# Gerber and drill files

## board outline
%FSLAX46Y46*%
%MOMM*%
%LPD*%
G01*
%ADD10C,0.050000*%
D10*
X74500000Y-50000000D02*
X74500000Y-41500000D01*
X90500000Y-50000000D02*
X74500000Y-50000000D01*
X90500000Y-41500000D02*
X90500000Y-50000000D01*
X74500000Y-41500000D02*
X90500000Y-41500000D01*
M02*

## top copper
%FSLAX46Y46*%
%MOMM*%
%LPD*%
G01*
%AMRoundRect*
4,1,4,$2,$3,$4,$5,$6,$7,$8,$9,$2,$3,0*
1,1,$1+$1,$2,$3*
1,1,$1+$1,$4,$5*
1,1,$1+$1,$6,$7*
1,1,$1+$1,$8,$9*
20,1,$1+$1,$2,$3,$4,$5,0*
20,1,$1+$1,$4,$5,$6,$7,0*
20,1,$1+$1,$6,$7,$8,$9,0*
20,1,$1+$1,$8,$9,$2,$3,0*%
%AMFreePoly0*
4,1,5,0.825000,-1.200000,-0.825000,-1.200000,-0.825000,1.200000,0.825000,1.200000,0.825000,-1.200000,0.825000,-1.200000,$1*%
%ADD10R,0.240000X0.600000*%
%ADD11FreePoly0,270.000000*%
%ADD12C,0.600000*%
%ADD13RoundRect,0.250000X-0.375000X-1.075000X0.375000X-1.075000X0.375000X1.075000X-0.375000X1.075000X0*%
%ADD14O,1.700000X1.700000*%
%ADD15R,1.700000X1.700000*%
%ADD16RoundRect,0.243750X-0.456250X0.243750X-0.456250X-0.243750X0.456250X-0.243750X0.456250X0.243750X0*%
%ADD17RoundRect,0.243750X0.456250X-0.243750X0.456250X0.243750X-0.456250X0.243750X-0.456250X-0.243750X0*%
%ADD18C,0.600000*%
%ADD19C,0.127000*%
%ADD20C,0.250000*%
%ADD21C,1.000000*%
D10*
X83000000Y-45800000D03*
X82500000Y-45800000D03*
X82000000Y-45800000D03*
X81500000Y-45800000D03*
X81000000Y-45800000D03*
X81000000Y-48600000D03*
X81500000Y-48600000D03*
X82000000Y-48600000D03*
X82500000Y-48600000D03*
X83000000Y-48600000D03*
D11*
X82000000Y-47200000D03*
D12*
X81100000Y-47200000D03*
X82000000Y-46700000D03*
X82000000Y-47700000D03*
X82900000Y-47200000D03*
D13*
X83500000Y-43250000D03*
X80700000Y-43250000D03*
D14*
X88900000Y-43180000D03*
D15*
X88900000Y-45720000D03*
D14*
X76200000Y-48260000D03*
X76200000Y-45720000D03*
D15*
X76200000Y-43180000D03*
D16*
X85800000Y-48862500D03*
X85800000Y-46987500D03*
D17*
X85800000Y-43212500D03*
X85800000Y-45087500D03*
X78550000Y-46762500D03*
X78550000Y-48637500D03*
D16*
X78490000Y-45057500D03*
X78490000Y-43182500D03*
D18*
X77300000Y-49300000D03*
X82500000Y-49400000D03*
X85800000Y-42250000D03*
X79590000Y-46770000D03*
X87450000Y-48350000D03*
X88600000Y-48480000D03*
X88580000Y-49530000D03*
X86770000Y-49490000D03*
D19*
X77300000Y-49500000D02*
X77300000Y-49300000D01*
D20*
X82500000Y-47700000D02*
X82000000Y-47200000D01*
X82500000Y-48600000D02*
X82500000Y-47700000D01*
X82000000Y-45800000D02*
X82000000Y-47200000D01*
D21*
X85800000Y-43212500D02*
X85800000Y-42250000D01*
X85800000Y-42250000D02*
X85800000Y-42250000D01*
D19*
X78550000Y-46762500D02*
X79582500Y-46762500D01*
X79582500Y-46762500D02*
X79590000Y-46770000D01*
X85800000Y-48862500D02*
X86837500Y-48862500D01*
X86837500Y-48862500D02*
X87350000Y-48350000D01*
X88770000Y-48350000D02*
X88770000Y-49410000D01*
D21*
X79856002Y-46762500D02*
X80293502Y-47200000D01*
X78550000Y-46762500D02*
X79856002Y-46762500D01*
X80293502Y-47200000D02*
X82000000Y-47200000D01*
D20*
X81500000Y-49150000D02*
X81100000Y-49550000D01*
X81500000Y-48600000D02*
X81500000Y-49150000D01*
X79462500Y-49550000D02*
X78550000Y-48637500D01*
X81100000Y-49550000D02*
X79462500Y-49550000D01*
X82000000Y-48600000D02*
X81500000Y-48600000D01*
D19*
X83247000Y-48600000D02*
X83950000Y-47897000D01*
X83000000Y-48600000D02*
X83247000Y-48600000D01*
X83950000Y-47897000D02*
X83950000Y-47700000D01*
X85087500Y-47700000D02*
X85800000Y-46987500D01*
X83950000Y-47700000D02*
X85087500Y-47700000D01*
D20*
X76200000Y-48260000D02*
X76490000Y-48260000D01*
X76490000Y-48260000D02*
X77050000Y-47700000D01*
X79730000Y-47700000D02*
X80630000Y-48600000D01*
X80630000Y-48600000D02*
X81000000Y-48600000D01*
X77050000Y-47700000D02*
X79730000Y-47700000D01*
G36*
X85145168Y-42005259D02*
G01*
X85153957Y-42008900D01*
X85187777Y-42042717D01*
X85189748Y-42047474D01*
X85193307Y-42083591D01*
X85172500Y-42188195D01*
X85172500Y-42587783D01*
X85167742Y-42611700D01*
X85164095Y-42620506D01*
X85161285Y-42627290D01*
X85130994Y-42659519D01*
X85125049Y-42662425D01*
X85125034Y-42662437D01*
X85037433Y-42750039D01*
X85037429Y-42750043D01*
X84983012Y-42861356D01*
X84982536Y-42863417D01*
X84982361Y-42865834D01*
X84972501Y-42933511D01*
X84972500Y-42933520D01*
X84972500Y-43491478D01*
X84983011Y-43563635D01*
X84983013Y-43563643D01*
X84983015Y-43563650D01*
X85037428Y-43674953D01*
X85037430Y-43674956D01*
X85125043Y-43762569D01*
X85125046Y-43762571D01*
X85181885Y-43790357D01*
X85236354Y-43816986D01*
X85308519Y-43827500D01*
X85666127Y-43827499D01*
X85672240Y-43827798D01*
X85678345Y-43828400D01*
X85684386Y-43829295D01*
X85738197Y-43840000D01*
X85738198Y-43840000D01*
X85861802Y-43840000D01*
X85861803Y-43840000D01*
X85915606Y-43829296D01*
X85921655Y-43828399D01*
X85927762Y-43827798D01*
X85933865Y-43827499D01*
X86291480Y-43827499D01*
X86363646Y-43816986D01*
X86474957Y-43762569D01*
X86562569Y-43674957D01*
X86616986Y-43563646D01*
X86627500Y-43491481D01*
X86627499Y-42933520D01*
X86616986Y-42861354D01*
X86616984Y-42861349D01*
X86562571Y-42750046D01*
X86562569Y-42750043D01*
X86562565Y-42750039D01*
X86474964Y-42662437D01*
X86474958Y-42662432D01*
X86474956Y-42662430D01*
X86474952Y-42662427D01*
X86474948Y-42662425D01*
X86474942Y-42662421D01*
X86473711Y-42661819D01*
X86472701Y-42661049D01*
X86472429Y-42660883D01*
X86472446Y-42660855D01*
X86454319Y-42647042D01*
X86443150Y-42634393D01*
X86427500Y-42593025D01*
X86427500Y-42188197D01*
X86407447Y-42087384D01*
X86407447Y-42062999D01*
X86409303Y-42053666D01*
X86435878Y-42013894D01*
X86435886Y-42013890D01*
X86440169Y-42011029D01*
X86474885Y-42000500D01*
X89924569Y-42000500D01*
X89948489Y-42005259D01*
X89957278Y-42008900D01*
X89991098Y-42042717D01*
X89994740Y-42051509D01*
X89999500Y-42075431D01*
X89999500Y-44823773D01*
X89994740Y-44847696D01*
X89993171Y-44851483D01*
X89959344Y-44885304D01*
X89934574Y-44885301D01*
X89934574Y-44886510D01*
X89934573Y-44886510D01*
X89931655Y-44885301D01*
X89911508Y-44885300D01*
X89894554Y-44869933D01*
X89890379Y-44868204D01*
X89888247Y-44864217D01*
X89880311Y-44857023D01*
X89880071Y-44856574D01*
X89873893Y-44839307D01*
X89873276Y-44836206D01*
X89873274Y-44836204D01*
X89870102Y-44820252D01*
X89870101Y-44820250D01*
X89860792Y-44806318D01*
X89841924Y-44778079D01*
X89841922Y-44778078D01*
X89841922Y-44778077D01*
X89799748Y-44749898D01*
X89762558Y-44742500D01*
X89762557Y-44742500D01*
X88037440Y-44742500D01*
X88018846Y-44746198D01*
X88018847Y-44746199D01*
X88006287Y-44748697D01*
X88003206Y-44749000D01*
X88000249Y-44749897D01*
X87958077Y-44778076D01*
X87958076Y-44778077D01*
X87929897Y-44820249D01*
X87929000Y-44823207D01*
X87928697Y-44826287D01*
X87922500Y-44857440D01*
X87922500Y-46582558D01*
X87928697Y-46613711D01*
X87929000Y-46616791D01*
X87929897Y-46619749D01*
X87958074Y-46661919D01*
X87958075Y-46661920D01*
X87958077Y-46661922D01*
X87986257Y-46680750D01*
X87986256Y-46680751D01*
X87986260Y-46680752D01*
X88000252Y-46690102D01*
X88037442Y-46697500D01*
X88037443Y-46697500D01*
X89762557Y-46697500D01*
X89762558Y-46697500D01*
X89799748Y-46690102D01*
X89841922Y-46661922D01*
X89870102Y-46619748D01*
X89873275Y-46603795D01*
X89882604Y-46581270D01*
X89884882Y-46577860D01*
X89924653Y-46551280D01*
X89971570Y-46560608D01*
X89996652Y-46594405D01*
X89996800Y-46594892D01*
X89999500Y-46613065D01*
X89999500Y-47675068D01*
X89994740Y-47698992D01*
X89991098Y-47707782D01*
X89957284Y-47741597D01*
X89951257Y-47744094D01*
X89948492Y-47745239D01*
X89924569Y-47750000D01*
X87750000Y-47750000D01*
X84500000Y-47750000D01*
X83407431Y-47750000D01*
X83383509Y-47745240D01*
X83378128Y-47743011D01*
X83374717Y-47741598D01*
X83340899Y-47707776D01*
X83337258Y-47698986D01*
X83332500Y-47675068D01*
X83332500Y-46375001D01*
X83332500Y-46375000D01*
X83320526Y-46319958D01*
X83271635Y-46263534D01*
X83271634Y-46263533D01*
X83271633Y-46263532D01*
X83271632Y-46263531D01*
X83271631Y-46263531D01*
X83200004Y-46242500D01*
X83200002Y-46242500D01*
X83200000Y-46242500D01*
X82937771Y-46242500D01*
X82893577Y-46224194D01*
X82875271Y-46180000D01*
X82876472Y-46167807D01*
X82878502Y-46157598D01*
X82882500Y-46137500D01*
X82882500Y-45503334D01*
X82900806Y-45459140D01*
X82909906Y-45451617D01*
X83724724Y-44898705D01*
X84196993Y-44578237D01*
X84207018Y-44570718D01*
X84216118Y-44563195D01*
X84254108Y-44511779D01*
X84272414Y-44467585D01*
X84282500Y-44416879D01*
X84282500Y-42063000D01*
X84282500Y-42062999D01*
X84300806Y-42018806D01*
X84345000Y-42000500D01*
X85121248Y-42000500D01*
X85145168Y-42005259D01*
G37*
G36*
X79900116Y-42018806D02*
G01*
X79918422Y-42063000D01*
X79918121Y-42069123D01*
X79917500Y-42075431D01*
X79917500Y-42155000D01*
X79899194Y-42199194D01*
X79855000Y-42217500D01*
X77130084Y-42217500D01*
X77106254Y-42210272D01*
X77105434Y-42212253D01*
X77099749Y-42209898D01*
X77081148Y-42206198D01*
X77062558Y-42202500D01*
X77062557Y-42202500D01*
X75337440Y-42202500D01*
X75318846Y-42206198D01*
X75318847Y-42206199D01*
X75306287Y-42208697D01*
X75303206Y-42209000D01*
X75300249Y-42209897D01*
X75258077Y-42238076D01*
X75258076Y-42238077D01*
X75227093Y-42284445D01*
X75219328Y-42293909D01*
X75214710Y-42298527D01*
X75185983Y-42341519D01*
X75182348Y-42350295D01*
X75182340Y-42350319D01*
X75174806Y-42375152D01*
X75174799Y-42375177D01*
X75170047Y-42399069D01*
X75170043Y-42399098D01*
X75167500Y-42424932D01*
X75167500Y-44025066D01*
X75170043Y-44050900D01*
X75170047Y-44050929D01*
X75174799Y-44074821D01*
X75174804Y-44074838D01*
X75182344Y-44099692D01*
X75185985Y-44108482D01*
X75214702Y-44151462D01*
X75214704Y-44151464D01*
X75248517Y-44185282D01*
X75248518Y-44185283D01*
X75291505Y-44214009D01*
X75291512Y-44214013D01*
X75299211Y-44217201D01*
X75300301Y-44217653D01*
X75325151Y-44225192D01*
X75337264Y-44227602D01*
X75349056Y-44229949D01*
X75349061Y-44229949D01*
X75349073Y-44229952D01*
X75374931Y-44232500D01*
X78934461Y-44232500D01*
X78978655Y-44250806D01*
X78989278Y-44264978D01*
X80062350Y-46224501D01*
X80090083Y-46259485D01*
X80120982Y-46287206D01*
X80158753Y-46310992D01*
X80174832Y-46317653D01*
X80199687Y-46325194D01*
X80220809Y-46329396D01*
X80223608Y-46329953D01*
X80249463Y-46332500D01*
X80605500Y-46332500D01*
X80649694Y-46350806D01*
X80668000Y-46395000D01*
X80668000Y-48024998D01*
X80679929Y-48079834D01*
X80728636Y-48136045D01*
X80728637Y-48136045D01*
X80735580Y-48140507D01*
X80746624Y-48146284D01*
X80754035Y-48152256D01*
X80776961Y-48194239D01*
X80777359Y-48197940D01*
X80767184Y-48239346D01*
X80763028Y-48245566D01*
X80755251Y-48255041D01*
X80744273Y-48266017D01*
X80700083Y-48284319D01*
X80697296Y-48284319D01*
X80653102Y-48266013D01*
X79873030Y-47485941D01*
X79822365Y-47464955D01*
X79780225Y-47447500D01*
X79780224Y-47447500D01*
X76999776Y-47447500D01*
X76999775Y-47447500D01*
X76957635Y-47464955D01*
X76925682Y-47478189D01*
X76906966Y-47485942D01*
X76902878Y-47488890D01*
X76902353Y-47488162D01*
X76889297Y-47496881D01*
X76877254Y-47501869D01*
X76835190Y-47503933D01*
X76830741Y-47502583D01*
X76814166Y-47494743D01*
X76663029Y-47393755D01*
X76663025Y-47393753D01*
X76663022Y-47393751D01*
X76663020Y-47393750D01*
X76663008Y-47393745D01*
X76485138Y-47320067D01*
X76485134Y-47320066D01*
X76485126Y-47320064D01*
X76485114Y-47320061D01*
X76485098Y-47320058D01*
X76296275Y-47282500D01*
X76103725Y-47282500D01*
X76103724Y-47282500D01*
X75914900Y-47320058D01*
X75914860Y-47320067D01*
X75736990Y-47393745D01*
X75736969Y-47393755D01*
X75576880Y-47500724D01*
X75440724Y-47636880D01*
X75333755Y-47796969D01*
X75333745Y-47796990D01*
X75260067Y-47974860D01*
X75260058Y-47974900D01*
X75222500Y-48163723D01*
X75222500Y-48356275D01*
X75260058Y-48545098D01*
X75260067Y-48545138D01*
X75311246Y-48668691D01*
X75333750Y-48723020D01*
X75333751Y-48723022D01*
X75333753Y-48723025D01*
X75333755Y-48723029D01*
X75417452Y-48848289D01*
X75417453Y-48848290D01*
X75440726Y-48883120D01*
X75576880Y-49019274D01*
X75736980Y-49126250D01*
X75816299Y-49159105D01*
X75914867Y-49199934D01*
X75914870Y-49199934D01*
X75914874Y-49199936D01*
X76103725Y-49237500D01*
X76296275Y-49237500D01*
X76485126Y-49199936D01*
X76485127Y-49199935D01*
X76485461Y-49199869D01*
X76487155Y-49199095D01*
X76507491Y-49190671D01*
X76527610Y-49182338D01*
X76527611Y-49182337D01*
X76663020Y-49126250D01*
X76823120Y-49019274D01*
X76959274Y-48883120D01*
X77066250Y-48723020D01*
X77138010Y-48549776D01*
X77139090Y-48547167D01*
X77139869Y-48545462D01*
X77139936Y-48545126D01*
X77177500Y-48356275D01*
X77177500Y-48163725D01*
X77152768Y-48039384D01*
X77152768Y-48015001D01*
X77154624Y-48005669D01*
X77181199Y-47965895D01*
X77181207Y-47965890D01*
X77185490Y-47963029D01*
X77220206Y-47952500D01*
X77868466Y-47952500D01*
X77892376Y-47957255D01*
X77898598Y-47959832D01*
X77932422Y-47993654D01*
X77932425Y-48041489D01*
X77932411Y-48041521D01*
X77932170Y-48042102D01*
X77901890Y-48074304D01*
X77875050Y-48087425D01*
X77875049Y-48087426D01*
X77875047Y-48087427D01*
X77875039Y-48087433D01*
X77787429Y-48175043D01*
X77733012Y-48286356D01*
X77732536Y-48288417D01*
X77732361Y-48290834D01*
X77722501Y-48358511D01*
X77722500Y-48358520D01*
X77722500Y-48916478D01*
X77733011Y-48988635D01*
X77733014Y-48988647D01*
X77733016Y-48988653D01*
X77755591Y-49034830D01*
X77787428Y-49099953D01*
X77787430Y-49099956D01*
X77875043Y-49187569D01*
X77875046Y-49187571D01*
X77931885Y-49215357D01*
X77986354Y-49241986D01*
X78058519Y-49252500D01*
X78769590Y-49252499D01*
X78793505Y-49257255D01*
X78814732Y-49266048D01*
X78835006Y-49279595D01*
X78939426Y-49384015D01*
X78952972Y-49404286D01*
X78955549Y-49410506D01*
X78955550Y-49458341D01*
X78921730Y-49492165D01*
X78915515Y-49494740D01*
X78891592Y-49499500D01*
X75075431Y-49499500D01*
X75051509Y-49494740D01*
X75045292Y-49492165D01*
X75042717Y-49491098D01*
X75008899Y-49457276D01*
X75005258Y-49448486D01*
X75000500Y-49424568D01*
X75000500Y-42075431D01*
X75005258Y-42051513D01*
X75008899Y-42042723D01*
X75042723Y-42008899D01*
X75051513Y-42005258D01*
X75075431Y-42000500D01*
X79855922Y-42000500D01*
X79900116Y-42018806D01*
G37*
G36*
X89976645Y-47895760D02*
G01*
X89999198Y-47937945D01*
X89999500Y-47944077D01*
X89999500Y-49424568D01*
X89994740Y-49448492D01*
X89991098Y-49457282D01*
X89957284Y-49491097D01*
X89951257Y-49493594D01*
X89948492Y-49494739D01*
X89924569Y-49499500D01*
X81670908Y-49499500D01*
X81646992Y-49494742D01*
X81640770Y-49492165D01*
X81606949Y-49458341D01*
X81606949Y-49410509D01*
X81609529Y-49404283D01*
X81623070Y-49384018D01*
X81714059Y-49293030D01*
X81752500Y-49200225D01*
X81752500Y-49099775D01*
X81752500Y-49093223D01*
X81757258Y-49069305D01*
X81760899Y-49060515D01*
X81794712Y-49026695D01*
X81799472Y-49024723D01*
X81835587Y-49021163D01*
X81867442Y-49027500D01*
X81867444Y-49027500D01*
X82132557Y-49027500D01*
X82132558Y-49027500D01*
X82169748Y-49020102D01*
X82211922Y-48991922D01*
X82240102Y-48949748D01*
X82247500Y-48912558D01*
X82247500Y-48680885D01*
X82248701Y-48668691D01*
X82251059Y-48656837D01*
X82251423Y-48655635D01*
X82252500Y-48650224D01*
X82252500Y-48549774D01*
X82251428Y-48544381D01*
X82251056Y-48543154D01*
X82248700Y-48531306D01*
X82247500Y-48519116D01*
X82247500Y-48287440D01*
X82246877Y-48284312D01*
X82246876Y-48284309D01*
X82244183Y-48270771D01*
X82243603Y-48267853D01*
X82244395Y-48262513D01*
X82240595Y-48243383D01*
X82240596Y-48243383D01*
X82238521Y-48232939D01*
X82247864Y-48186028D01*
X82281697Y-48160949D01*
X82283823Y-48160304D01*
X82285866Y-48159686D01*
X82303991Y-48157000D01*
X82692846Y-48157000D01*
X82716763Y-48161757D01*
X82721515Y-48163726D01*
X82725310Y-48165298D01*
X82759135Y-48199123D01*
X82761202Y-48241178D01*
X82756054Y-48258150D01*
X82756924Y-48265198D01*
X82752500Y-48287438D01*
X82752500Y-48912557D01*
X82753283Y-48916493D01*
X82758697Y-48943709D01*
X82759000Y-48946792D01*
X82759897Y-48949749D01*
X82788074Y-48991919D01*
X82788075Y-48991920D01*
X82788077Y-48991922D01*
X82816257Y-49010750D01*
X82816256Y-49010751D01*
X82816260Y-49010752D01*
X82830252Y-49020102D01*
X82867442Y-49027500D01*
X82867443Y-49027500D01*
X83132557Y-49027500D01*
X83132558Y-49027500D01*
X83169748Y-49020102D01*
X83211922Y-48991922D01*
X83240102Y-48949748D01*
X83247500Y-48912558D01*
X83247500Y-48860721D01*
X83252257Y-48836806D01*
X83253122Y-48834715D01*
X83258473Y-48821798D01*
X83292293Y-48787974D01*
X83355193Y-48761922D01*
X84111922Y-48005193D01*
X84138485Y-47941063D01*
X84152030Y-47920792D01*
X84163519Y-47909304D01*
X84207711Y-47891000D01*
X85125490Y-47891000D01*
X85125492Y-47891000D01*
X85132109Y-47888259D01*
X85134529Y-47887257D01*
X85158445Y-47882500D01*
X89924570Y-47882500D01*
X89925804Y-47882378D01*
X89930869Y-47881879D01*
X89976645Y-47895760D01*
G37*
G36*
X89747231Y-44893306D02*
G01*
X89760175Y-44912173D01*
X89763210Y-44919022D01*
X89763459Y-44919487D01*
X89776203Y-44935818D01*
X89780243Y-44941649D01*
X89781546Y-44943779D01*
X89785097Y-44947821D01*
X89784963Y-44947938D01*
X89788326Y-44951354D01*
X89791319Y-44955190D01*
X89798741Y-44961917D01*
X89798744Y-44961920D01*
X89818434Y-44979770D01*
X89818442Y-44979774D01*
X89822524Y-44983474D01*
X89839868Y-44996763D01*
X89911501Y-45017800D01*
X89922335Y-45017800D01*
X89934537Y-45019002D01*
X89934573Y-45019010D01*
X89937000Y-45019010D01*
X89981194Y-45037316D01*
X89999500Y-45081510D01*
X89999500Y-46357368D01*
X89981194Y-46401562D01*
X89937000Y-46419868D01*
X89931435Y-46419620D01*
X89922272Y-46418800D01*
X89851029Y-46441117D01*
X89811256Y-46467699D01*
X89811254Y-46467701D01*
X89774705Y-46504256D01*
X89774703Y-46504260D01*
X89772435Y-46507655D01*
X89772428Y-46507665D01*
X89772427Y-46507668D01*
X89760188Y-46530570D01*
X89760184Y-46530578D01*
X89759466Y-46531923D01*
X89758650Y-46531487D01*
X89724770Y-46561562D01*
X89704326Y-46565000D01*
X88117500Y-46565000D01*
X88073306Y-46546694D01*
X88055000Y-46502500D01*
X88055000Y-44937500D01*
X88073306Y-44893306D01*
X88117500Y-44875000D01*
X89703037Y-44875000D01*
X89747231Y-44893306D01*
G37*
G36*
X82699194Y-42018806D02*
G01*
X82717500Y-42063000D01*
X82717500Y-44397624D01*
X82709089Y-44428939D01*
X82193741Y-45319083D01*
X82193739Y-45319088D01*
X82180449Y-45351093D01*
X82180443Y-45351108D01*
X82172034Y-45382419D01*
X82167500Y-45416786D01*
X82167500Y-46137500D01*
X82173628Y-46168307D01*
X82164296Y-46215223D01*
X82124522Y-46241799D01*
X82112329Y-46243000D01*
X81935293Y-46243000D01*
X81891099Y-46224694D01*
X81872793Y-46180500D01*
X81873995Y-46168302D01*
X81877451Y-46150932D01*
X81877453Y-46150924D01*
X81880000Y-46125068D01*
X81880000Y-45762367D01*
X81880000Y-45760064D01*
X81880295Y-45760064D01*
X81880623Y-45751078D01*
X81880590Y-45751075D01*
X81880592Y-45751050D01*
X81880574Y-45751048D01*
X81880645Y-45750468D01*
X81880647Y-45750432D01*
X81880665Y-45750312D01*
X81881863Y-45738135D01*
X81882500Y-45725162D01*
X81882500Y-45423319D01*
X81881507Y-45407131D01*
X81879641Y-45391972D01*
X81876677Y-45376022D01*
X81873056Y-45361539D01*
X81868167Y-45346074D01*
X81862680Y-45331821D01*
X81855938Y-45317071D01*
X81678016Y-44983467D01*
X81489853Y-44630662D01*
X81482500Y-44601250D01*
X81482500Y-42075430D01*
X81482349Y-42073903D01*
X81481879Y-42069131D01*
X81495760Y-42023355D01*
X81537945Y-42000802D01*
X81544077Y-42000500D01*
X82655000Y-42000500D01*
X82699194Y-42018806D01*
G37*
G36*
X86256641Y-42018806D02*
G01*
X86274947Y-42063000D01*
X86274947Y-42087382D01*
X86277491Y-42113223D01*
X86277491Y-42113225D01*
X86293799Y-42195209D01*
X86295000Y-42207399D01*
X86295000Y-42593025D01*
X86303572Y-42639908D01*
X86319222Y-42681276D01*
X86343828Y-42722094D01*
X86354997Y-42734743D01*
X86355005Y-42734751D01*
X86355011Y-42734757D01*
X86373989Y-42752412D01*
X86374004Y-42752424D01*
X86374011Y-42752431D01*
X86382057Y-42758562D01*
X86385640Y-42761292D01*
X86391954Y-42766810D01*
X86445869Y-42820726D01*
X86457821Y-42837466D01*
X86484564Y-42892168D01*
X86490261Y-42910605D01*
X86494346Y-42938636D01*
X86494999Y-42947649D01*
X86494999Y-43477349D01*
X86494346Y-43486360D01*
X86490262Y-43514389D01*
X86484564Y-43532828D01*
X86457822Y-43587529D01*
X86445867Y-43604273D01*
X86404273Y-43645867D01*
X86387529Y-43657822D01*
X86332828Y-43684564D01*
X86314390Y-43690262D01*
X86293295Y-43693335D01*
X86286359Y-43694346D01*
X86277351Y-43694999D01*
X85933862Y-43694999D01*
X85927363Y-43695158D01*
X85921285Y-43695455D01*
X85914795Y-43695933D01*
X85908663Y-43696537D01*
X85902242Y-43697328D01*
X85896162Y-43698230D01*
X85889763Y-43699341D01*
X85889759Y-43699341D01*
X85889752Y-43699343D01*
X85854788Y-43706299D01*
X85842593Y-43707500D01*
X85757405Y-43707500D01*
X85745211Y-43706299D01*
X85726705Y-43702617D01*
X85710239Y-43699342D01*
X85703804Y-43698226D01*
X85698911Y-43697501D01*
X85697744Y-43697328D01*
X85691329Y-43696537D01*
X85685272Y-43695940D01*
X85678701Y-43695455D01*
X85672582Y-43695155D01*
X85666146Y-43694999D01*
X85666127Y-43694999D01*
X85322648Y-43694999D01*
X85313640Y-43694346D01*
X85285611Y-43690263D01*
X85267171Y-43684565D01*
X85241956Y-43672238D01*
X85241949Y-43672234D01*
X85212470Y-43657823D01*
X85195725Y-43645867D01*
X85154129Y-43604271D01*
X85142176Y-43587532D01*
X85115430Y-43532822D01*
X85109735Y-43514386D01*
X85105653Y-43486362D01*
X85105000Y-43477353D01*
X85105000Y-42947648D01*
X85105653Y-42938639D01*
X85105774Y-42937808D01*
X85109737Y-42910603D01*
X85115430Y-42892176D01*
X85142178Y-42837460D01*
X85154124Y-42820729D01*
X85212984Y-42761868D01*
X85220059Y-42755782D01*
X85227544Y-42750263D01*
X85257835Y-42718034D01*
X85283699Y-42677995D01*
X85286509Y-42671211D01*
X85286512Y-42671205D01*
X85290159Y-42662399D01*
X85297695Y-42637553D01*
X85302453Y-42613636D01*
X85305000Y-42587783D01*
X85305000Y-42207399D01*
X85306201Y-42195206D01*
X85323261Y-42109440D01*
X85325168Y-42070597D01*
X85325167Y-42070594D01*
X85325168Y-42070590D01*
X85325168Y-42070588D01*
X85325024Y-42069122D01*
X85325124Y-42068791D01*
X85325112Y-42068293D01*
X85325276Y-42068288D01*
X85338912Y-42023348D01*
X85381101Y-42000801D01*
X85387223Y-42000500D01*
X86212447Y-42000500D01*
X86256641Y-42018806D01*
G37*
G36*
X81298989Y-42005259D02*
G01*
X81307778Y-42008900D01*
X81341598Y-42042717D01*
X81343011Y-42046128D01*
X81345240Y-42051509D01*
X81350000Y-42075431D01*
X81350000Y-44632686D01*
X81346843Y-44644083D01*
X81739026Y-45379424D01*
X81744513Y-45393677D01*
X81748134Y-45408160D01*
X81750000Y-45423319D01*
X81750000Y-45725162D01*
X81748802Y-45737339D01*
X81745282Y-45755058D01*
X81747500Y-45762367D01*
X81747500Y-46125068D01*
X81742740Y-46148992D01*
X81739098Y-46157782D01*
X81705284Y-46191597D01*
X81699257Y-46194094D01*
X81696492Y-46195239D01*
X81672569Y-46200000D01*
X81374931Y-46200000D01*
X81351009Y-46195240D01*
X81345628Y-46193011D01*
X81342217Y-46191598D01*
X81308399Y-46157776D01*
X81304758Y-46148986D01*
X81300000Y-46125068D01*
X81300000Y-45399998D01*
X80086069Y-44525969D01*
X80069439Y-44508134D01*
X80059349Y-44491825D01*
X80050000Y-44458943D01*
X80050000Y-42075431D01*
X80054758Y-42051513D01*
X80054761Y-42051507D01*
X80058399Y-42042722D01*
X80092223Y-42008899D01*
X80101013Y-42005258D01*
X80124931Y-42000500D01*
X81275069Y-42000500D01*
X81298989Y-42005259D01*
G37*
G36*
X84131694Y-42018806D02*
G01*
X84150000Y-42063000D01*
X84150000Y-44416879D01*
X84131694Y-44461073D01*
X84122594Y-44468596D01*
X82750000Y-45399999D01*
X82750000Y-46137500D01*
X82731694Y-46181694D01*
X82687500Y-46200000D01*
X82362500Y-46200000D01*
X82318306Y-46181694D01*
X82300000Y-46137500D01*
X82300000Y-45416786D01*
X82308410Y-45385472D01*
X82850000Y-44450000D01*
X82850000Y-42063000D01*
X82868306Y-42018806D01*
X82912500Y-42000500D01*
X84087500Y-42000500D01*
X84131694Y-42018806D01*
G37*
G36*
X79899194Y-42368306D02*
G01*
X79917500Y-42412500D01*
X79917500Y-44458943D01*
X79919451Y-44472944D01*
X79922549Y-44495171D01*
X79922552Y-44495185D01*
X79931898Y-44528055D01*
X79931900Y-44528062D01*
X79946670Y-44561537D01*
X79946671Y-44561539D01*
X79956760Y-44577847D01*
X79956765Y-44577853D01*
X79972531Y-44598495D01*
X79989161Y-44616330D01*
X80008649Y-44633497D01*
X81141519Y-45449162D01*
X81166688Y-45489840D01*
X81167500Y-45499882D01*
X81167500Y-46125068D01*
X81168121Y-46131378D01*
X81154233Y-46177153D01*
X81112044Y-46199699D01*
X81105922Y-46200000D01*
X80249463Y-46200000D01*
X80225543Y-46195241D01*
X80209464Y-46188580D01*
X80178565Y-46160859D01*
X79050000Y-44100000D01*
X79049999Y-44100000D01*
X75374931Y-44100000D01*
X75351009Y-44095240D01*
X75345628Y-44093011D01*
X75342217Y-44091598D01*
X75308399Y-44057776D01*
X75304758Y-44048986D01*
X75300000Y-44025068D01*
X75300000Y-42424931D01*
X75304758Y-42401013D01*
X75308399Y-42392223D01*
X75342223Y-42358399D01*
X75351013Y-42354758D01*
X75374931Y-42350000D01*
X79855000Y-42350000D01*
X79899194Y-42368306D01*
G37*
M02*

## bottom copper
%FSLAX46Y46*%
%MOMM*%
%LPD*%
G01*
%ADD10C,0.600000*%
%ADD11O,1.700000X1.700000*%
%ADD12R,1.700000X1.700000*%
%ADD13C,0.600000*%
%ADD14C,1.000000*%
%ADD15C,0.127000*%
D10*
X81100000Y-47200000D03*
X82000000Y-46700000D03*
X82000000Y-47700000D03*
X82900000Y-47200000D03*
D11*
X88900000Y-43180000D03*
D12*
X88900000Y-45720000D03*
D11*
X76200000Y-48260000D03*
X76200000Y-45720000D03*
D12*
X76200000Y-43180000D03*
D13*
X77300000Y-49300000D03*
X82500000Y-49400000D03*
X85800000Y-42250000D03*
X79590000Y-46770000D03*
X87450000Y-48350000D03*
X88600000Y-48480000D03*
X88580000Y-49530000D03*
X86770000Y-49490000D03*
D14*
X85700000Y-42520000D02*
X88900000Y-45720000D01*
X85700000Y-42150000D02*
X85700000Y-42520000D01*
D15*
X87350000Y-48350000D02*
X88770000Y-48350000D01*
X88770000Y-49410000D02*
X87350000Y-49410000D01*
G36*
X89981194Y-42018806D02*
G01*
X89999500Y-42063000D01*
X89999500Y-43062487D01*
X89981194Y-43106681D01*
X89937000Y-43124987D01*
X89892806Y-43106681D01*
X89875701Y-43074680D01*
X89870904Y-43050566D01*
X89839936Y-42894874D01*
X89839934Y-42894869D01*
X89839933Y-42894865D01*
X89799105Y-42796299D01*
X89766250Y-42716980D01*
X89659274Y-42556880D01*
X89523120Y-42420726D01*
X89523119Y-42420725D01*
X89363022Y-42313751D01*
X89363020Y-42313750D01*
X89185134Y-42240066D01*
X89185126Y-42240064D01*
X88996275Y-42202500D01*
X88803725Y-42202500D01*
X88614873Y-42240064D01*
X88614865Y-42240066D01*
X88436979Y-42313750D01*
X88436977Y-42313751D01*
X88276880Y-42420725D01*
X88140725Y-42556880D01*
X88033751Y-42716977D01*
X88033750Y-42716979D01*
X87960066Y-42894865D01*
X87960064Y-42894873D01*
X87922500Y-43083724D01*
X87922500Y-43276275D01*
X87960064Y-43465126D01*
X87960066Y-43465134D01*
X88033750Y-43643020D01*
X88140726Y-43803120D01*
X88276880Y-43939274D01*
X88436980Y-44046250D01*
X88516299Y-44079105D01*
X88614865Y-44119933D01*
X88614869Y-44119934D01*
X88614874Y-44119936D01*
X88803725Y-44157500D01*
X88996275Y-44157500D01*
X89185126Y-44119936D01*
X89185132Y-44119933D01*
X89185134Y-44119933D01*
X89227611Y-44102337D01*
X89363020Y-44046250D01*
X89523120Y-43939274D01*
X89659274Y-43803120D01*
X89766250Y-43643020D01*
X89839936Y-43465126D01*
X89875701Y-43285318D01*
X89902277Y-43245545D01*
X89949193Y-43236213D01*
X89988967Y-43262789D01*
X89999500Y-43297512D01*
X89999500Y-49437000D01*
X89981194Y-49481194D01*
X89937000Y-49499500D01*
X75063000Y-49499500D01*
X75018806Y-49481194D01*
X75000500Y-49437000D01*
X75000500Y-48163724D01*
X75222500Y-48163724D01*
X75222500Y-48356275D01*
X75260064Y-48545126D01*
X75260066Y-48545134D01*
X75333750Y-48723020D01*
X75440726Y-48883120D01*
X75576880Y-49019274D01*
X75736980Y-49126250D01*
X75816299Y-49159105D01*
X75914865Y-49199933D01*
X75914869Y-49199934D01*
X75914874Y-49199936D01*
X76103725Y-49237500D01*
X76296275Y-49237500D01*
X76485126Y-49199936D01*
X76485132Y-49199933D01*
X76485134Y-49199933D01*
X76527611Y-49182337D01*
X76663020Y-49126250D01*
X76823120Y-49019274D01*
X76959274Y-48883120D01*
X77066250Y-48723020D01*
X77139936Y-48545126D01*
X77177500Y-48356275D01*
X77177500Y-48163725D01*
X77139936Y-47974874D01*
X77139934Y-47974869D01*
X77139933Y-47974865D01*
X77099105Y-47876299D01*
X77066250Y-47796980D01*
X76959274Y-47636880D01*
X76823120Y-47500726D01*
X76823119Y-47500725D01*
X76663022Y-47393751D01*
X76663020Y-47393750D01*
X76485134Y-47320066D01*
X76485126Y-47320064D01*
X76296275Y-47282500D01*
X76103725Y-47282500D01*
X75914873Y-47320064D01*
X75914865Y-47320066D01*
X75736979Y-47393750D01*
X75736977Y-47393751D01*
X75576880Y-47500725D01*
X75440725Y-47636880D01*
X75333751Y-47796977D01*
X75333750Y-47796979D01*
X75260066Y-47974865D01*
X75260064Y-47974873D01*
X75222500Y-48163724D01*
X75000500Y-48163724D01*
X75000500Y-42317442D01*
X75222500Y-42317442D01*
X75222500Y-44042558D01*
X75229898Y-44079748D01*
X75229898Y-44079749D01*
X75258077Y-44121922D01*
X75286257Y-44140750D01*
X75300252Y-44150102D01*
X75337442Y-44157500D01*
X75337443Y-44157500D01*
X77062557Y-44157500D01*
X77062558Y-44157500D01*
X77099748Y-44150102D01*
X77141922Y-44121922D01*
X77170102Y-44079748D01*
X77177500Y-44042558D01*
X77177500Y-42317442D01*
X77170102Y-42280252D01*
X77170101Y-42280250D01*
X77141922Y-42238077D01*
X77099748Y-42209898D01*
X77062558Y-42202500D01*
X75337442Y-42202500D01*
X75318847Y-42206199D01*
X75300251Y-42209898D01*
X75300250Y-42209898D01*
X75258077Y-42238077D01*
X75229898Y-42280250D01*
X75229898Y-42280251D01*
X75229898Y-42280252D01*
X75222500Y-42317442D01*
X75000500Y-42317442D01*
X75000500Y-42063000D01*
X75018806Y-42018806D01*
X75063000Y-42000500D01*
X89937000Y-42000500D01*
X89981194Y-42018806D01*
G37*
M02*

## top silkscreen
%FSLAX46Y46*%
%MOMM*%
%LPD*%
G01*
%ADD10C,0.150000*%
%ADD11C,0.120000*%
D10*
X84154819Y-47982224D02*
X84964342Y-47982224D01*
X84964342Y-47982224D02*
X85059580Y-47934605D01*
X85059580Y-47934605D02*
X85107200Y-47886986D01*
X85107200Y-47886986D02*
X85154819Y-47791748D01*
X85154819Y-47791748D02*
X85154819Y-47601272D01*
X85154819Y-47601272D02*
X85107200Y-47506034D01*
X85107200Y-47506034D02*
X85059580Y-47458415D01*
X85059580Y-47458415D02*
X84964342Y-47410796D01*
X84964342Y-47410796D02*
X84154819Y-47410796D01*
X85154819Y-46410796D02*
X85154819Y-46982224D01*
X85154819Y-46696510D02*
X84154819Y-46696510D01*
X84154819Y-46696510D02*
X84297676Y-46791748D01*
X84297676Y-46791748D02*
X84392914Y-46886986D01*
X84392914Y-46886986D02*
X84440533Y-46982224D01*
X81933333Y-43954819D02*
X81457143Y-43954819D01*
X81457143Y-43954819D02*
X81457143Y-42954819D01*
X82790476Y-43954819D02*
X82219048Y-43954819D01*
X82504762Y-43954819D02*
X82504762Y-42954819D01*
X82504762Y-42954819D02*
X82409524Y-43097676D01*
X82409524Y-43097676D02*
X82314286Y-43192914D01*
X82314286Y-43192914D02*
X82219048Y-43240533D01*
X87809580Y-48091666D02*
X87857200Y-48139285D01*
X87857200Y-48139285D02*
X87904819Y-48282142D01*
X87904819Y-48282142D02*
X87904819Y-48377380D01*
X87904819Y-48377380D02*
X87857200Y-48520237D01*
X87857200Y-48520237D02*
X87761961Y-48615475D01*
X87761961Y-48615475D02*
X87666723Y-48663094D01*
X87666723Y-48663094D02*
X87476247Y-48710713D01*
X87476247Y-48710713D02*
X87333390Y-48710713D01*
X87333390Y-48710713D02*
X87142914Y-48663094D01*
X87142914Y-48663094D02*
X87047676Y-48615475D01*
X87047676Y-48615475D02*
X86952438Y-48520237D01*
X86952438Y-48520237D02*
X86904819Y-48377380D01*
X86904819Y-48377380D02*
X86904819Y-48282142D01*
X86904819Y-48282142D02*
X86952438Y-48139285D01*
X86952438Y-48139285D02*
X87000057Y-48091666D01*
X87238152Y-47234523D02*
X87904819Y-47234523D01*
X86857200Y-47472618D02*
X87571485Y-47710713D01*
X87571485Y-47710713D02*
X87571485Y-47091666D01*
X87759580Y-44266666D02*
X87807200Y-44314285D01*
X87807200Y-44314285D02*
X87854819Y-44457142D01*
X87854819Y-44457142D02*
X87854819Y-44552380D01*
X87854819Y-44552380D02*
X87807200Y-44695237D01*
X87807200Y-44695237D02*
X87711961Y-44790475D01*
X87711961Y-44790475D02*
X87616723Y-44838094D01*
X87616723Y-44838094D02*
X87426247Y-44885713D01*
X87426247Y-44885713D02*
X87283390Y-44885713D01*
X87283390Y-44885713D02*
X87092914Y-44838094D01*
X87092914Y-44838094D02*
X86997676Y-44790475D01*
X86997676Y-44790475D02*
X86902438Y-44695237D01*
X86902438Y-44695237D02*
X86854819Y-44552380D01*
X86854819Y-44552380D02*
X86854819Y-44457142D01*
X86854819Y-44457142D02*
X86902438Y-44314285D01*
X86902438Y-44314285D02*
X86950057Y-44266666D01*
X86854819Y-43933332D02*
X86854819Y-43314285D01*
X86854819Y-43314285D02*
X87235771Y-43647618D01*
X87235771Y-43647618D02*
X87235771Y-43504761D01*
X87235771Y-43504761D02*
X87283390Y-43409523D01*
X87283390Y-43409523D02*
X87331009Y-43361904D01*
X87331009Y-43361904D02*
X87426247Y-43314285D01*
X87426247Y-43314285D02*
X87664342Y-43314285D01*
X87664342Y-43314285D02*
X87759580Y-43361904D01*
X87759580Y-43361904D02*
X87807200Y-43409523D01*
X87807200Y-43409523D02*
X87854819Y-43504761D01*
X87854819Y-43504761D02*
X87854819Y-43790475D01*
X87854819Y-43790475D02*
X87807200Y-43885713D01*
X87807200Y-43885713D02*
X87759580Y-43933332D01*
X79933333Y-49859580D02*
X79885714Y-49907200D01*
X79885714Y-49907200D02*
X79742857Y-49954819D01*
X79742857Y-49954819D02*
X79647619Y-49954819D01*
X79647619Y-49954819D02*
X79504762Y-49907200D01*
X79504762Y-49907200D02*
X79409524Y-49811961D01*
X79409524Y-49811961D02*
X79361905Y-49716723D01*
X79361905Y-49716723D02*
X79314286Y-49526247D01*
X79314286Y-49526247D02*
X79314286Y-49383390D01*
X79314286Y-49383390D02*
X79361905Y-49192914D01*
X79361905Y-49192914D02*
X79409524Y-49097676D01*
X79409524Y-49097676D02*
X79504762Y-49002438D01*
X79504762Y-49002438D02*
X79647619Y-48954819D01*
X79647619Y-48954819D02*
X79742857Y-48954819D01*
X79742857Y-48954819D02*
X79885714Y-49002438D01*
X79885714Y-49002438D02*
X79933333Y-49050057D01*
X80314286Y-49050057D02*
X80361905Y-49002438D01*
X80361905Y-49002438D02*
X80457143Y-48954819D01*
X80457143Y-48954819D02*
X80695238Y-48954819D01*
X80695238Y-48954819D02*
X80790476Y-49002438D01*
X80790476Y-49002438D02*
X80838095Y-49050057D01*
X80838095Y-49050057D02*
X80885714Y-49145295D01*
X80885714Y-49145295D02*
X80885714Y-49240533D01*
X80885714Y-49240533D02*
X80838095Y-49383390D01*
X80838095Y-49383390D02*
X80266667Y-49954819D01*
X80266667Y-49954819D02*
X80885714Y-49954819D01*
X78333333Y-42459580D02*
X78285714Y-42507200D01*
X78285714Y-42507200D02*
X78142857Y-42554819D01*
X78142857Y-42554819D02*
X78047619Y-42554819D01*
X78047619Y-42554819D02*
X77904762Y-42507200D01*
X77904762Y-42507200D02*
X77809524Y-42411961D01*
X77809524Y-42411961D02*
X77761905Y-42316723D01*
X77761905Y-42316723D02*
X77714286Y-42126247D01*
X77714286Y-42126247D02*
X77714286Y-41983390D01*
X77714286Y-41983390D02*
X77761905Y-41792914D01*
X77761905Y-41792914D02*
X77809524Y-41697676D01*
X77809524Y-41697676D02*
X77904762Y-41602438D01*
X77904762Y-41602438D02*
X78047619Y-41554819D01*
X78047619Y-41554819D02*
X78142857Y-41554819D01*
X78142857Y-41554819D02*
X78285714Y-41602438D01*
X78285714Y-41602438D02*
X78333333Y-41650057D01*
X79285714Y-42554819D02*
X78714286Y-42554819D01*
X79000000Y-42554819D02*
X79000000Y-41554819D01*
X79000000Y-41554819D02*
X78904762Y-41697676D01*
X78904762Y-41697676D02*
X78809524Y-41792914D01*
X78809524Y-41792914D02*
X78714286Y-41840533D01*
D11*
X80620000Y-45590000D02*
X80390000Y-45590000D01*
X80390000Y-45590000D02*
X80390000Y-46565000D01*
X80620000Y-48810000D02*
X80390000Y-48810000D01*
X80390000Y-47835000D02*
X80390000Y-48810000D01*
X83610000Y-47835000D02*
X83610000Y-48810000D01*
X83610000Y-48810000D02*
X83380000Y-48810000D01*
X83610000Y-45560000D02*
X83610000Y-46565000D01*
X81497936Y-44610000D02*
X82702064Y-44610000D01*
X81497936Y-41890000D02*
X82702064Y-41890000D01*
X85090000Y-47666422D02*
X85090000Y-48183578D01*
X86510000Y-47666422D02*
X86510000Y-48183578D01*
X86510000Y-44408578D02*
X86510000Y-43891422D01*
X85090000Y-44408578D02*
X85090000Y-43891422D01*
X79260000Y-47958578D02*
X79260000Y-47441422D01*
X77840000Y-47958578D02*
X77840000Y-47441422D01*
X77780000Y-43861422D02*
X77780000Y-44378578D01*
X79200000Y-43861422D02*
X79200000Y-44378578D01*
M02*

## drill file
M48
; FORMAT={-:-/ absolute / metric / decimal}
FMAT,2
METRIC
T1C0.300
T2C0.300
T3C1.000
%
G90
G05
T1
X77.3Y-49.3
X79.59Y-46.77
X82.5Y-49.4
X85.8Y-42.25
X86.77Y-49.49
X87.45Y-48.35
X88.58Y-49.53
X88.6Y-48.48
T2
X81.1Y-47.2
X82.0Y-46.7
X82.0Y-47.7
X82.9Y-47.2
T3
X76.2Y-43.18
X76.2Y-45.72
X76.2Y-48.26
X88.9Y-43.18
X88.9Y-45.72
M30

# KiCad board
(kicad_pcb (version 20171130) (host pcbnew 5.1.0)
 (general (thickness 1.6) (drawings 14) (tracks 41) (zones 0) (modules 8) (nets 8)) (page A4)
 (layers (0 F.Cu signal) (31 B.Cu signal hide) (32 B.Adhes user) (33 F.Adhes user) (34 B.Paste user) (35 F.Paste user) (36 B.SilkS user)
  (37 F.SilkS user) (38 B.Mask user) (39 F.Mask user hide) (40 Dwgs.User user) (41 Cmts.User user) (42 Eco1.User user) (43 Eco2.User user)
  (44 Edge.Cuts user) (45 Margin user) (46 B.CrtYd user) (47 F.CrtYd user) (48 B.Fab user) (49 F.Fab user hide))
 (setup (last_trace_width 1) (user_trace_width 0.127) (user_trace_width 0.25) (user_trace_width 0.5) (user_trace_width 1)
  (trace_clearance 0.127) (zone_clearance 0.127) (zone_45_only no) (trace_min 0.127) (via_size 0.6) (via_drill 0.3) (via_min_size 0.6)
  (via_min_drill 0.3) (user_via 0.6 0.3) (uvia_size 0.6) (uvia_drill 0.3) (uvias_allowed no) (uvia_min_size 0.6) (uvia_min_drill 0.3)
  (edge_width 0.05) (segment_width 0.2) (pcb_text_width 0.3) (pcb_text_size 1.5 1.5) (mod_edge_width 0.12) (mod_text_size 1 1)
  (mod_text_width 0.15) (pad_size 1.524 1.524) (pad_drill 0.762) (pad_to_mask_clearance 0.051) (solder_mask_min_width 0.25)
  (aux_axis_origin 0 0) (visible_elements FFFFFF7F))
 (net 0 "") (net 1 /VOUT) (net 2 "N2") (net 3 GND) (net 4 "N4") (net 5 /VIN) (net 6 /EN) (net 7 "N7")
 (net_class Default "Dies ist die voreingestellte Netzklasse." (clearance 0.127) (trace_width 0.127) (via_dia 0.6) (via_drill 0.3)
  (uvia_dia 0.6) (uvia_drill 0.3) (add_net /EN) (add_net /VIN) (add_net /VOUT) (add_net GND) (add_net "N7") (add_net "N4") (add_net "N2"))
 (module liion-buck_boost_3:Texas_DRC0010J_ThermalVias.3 (layer F.Cu) (at 82 47.2 270)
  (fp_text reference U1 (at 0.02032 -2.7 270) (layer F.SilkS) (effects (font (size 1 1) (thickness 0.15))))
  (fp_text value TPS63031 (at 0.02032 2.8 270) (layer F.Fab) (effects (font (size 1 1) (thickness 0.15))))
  (fp_line (start -1.61 1.38) (end -1.61 1.61) (layer F.SilkS) (width 0.12))
  (fp_line (start -1.61 1.61) (end -0.635 1.61) (layer F.SilkS) (width 0.12))
  (fp_line (start 1.61 1.38) (end 1.61 1.61) (layer F.SilkS) (width 0.12))
  (fp_line (start 0.635 1.61) (end 1.61 1.61) (layer F.SilkS) (width 0.12))
  (fp_line (start 0.635 -1.61) (end 1.61 -1.61) (layer F.SilkS) (width 0.12))
  (fp_line (start 1.61 -1.61) (end 1.61 -1.38) (layer F.SilkS) (width 0.12))
  (fp_line (start -1.64 -1.61) (end -0.635 -1.61) (layer F.SilkS) (width 0.12))
  (pad "" smd roundrect (at 0 0.63 270) (size 1.5 1.06) (layers F.Paste) (roundrect_rratio 0.1) (zone_connect 0))
  (pad "" smd roundrect (at 0 -0.63 270) (size 1.5 1.06) (layers F.Paste) (roundrect_rratio 0.1) (zone_connect 0))
  (pad "" smd roundrect (at -0.25 -1.53 270) (size 0.25 0.34) (layers F.Paste) (roundrect_rratio 0.1) (zone_connect 0))
  (pad "" smd roundrect (at 0.25 -1.53 270) (size 0.25 0.34) (layers F.Paste) (roundrect_rratio 0.1) (zone_connect 0))
  (pad "" smd roundrect (at -0.25 1.53 270) (size 0.25 0.34) (layers F.Paste) (roundrect_rratio 0.1) (zone_connect 0))
  (pad "" smd roundrect (at 0.25 1.53 270) (size 0.25 0.34) (layers F.Paste) (roundrect_rratio 0.1) (zone_connect 0))
  (pad 1 smd rect (at -1.4 -1 270) (size 0.6 0.24) (layers F.Cu F.Paste F.Mask) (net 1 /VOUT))
  (pad 2 smd rect (at -1.4 -0.5 270) (size 0.6 0.24) (layers F.Cu F.Paste F.Mask) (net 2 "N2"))
  (pad 3 smd rect (at -1.4 0 270) (size 0.6 0.24) (layers F.Cu F.Paste F.Mask) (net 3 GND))
  (pad 4 smd rect (at -1.4 0.5 270) (size 0.6 0.24) (layers F.Cu F.Paste F.Mask) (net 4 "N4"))
  (pad 5 smd rect (at -1.4 1 270) (size 0.6 0.24) (layers F.Cu F.Paste F.Mask) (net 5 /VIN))
  (pad 6 smd rect (at 1.4 1 270) (size 0.6 0.24) (layers F.Cu F.Paste F.Mask) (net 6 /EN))
  (pad 7 smd rect (at 1.4 0.5 270) (size 0.6 0.24) (layers F.Cu F.Paste F.Mask) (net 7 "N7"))
  (pad 8 smd rect (at 1.4 0 270) (size 0.6 0.24) (layers F.Cu F.Paste F.Mask) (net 7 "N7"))
  (pad 9 smd rect (at 1.4 -0.5 270) (size 0.6 0.24) (layers F.Cu F.Paste F.Mask) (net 3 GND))
  (pad 10 smd rect (at 1.4 -1 270) (size 0.6 0.24) (layers F.Cu F.Paste F.Mask) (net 1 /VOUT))
  (pad 11 smd custom (at 0 0 270) (size 1.65 2.4) (layers F.Cu F.Mask) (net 3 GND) (zone_connect 0)
   (options (clearance outline) (anchor rect)) (primitives))
  (pad 11 thru_hole circle (at 0 0.9 270) (size 0.6 0.6) (drill 0.3) (layers *.Cu) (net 3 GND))
  (pad 11 thru_hole circle (at -0.5 0 270) (size 0.6 0.6) (drill 0.3) (layers *.Cu) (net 3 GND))
  (pad 11 thru_hole circle (at 0.5 0 270) (size 0.6 0.6) (drill 0.3) (layers *.Cu) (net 3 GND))
  (pad 11 thru_hole circle (at 0 -0.9 270) (size 0.6 0.6) (drill 0.3) (layers *.Cu) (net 3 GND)))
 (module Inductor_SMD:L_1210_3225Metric (layer F.Cu) (at 82.1 43.25)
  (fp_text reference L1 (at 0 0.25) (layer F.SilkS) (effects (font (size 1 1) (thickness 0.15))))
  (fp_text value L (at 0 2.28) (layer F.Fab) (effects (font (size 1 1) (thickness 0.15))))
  (fp_line (start -0.602064 1.36) (end 0.602064 1.36) (layer F.SilkS) (width 0.12))
  (fp_line (start -0.602064 -1.36) (end 0.602064 -1.36) (layer F.SilkS) (width 0.12))
  (pad 2 smd roundrect (at 1.4 0) (size 1.25 2.65) (layers F.Cu F.Paste F.Mask) (roundrect_rratio 0.2) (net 2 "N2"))
  (pad 1 smd roundrect (at -1.4 0) (size 1.25 2.65) (layers F.Cu F.Paste F.Mask) (roundrect_rratio 0.2) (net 4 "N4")))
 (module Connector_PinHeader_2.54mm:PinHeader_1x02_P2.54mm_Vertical (layer B.Cu) (at 88.9 45.72)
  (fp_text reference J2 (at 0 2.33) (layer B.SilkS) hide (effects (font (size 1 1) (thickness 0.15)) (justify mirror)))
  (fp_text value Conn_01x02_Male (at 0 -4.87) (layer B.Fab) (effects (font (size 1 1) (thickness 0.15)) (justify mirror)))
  (pad 2 thru_hole oval (at 0 -2.54) (size 1.7 1.7) (drill 1) (layers *.Cu *.Mask) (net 1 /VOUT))
  (pad 1 thru_hole rect (at 0 0) (size 1.7 1.7) (drill 1) (layers *.Cu *.Mask) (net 3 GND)))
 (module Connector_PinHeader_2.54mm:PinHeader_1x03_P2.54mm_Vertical (layer B.Cu) (at 76.2 43.18 180)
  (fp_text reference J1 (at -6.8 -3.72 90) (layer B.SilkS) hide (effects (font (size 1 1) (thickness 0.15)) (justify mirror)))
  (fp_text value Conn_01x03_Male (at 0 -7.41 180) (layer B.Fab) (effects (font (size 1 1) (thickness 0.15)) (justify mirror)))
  (pad 3 thru_hole oval (at 0 -5.08 180) (size 1.7 1.7) (drill 1) (layers *.Cu *.Mask) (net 6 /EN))
  (pad 2 thru_hole oval (at 0 -2.54 180) (size 1.7 1.7) (drill 1) (layers *.Cu *.Mask) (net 3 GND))
  (pad 1 thru_hole rect (at 0 0 180) (size 1.7 1.7) (drill 1) (layers *.Cu *.Mask) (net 5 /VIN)))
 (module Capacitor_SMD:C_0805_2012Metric (layer F.Cu) (at 85.8 47.925 270)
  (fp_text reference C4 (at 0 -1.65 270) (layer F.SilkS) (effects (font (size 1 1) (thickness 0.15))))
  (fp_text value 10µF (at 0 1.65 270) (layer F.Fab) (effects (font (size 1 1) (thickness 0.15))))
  (fp_line (start -0.258578 0.71) (end 0.258578 0.71) (layer F.SilkS) (width 0.12))
  (fp_line (start -0.258578 -0.71) (end 0.258578 -0.71) (layer F.SilkS) (width 0.12))
  (pad 2 smd roundrect (at 0.9375 0 270) (size 0.975 1.4) (layers F.Cu F.Paste F.Mask) (roundrect_rratio 0.25) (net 3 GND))
  (pad 1 smd roundrect (at -0.9375 0 270) (size 0.975 1.4) (layers F.Cu F.Paste F.Mask) (roundrect_rratio 0.25) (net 1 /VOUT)))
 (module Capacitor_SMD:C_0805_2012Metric (layer F.Cu) (at 85.8 44.15 90)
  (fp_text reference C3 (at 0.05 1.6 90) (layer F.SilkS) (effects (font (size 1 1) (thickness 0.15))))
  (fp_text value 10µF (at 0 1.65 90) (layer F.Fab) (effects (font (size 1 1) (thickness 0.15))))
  (fp_line (start -0.258578 0.71) (end 0.258578 0.71) (layer F.SilkS) (width 0.12))
  (fp_line (start -0.258578 -0.71) (end 0.258578 -0.71) (layer F.SilkS) (width 0.12))
  (pad 2 smd roundrect (at 0.9375 0 90) (size 0.975 1.4) (layers F.Cu F.Paste F.Mask) (roundrect_rratio 0.25) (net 3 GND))
  (pad 1 smd roundrect (at -0.9375 0 90) (size 0.975 1.4) (layers F.Cu F.Paste F.Mask) (roundrect_rratio 0.25) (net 1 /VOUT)))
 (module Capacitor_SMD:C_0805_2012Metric (layer F.Cu) (at 78.55 47.7 90)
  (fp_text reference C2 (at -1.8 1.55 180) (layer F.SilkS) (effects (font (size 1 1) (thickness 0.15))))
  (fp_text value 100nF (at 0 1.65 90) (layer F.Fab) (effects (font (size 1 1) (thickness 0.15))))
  (fp_line (start -0.258578 0.71) (end 0.258578 0.71) (layer F.SilkS) (width 0.12))
  (fp_line (start -0.258578 -0.71) (end 0.258578 -0.71) (layer F.SilkS) (width 0.12))
  (pad 2 smd roundrect (at 0.9375 0 90) (size 0.975 1.4) (layers F.Cu F.Paste F.Mask) (roundrect_rratio 0.25) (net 3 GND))
  (pad 1 smd roundrect (at -0.9375 0 90) (size 0.975 1.4) (layers F.Cu F.Paste F.Mask) (roundrect_rratio 0.25) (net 7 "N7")))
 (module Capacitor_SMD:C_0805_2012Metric (layer F.Cu) (at 78.49 44.12 270)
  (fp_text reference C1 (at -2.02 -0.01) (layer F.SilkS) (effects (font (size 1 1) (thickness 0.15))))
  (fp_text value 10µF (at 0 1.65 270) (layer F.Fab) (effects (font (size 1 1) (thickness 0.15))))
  (fp_line (start -0.258578 0.71) (end 0.258578 0.71) (layer F.SilkS) (width 0.12))
  (fp_line (start -0.258578 -0.71) (end 0.258578 -0.71) (layer F.SilkS) (width 0.12))
  (pad 2 smd roundrect (at 0.9375 0 270) (size 0.975 1.4) (layers F.Cu F.Paste F.Mask) (roundrect_rratio 0.25) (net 3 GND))
  (pad 1 smd roundrect (at -0.9375 0 270) (size 0.975 1.4) (layers F.Cu F.Paste F.Mask) (roundrect_rratio 0.25) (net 5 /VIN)))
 (gr_line (start 74.5 50) (end 74.5 41.5) (layer Edge.Cuts) (width 0.05))
 (gr_line (start 90.5 50) (end 74.5 50) (layer Edge.Cuts) (width 0.05))
 (gr_line (start 90.5 41.5) (end 90.5 50) (layer Edge.Cuts) (width 0.05))
 (gr_line (start 74.5 41.5) (end 90.5 41.5) (layer Edge.Cuts) (width 0.05))
 (via (at 77.3 49.3) (size 0.6) (drill 0.3) (layers F.Cu B.Cu) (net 3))
 (segment (start 77.3 49.5) (end 77.3 49.3) (width 0.127) (layer F.Cu) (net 3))
 (via (at 82.5 49.4) (size 0.6) (drill 0.3) (layers F.Cu B.Cu) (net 3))
 (segment (start 82.5 47.7) (end 82 47.2) (width 0.25) (layer F.Cu) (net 3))
 (segment (start 82.5 48.6) (end 82.5 47.7) (width 0.25) (layer F.Cu) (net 3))
 (segment (start 82 45.8) (end 82 47.2) (width 0.25) (layer F.Cu) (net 3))
 (segment (start 85.8 43.2125) (end 85.8 42.25) (width 1) (layer F.Cu) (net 3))
 (segment (start 85.7 42.52) (end 88.9 45.72) (width 1) (layer B.Cu) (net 3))
 (segment (start 85.7 42.15) (end 85.7 42.52) (width 1) (layer B.Cu) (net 3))
 (segment (start 85.8 42.25) (end 85.8 42.25) (width 1) (layer F.Cu) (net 3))
 (via (at 85.8 42.25) (size 0.6) (drill 0.3) (layers F.Cu B.Cu) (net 3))
 (segment (start 78.55 46.7625) (end 79.5825 46.7625) (width 0.127) (layer F.Cu) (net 3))
 (via (at 79.59 46.77) (size 0.6) (drill 0.3) (layers F.Cu B.Cu) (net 3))
 (segment (start 79.5825 46.7625) (end 79.59 46.77) (width 0.127) (layer F.Cu) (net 3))
 (segment (start 85.8 48.8625) (end 86.8375 48.8625) (width 0.127) (layer F.Cu) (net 3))
 (via (at 87.45 48.35) (size 0.6) (drill 0.3) (layers F.Cu B.Cu) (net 3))
 (segment (start 86.8375 48.8625) (end 87.35 48.35) (width 0.127) (layer F.Cu) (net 3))
 (via (at 88.6 48.48) (size 0.6) (drill 0.3) (layers F.Cu B.Cu) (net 3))
 (segment (start 87.35 48.35) (end 88.77 48.35) (width 0.127) (layer B.Cu) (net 3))
 (via (at 88.58 49.53) (size 0.6) (drill 0.3) (layers F.Cu B.Cu) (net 3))
 (segment (start 88.77 48.35) (end 88.77 49.41) (width 0.127) (layer F.Cu) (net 3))
 (via (at 86.77 49.49) (size 0.6) (drill 0.3) (layers F.Cu B.Cu) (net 3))
 (segment (start 88.77 49.41) (end 87.35 49.41) (width 0.127) (layer B.Cu) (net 3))
 (segment (start 79.856002 46.7625) (end 80.293502 47.2) (width 1) (layer F.Cu) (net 3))
 (segment (start 78.55 46.7625) (end 79.856002 46.7625) (width 1) (layer F.Cu) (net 3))
 (segment (start 80.293502 47.2) (end 82 47.2) (width 1) (layer F.Cu) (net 3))
 (segment (start 81.5 49.15) (end 81.1 49.55) (width 0.25) (layer F.Cu) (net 7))
 (segment (start 81.5 48.6) (end 81.5 49.15) (width 0.25) (layer F.Cu) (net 7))
 (segment (start 79.4625 49.55) (end 78.55 48.6375) (width 0.25) (layer F.Cu) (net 7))
 (segment (start 81.1 49.55) (end 79.4625 49.55) (width 0.25) (layer F.Cu) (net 7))
 (segment (start 82 48.6) (end 81.5 48.6) (width 0.25) (layer F.Cu) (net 7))
 (segment (start 83.247 48.6) (end 83.95 47.897) (width 0.127) (layer F.Cu) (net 1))
 (segment (start 83 48.6) (end 83.247 48.6) (width 0.127) (layer F.Cu) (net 1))
 (segment (start 83.95 47.897) (end 83.95 47.7) (width 0.127) (layer F.Cu) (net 1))
 (segment (start 85.0875 47.7) (end 85.8 46.9875) (width 0.127) (layer F.Cu) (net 1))
 (segment (start 83.95 47.7) (end 85.0875 47.7) (width 0.127) (layer F.Cu) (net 1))
 (segment (start 76.2 48.26) (end 76.49 48.26) (width 0.25) (layer F.Cu) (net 6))
 (segment (start 76.49 48.26) (end 77.05 47.7) (width 0.25) (layer F.Cu) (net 6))
 (segment (start 79.73 47.7) (end 80.63 48.6) (width 0.25) (layer F.Cu) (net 6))
 (segment (start 80.63 48.6) (end 81 48.6) (width 0.25) (layer F.Cu) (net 6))
 (segment (start 77.05 47.7) (end 79.73 47.7) (width 0.25) (layer F.Cu) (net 6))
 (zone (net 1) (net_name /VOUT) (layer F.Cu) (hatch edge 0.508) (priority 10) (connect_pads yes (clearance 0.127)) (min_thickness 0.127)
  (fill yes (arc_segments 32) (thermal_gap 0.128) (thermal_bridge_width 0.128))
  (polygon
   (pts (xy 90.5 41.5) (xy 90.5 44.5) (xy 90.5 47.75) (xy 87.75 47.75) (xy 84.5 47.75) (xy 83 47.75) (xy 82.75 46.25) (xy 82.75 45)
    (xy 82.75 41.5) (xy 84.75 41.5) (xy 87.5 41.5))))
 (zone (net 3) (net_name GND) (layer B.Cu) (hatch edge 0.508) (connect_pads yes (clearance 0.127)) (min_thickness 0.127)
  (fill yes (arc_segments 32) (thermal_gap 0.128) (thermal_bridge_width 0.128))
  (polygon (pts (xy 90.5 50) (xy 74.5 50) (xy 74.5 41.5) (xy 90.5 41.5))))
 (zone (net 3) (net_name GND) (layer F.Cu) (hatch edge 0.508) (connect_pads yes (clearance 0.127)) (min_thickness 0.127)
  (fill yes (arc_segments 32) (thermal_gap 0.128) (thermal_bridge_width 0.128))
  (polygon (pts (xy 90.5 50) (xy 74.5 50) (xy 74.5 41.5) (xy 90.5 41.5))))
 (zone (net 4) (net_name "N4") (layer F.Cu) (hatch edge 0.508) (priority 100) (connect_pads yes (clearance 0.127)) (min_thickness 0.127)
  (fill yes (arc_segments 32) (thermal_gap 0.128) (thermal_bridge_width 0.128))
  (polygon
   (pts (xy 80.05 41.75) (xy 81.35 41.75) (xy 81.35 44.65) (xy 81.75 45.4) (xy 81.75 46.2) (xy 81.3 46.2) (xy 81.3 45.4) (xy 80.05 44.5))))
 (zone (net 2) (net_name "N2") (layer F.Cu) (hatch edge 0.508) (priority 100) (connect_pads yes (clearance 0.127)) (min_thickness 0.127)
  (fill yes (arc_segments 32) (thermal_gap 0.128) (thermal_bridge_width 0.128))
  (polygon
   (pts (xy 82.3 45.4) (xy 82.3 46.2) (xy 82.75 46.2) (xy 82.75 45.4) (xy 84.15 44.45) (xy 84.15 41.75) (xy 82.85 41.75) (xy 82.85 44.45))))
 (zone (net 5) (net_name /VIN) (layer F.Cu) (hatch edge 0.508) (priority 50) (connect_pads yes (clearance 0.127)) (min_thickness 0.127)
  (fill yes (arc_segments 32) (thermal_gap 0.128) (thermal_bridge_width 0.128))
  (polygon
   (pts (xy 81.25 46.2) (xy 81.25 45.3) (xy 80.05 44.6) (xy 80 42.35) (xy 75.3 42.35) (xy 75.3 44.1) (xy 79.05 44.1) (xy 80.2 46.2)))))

